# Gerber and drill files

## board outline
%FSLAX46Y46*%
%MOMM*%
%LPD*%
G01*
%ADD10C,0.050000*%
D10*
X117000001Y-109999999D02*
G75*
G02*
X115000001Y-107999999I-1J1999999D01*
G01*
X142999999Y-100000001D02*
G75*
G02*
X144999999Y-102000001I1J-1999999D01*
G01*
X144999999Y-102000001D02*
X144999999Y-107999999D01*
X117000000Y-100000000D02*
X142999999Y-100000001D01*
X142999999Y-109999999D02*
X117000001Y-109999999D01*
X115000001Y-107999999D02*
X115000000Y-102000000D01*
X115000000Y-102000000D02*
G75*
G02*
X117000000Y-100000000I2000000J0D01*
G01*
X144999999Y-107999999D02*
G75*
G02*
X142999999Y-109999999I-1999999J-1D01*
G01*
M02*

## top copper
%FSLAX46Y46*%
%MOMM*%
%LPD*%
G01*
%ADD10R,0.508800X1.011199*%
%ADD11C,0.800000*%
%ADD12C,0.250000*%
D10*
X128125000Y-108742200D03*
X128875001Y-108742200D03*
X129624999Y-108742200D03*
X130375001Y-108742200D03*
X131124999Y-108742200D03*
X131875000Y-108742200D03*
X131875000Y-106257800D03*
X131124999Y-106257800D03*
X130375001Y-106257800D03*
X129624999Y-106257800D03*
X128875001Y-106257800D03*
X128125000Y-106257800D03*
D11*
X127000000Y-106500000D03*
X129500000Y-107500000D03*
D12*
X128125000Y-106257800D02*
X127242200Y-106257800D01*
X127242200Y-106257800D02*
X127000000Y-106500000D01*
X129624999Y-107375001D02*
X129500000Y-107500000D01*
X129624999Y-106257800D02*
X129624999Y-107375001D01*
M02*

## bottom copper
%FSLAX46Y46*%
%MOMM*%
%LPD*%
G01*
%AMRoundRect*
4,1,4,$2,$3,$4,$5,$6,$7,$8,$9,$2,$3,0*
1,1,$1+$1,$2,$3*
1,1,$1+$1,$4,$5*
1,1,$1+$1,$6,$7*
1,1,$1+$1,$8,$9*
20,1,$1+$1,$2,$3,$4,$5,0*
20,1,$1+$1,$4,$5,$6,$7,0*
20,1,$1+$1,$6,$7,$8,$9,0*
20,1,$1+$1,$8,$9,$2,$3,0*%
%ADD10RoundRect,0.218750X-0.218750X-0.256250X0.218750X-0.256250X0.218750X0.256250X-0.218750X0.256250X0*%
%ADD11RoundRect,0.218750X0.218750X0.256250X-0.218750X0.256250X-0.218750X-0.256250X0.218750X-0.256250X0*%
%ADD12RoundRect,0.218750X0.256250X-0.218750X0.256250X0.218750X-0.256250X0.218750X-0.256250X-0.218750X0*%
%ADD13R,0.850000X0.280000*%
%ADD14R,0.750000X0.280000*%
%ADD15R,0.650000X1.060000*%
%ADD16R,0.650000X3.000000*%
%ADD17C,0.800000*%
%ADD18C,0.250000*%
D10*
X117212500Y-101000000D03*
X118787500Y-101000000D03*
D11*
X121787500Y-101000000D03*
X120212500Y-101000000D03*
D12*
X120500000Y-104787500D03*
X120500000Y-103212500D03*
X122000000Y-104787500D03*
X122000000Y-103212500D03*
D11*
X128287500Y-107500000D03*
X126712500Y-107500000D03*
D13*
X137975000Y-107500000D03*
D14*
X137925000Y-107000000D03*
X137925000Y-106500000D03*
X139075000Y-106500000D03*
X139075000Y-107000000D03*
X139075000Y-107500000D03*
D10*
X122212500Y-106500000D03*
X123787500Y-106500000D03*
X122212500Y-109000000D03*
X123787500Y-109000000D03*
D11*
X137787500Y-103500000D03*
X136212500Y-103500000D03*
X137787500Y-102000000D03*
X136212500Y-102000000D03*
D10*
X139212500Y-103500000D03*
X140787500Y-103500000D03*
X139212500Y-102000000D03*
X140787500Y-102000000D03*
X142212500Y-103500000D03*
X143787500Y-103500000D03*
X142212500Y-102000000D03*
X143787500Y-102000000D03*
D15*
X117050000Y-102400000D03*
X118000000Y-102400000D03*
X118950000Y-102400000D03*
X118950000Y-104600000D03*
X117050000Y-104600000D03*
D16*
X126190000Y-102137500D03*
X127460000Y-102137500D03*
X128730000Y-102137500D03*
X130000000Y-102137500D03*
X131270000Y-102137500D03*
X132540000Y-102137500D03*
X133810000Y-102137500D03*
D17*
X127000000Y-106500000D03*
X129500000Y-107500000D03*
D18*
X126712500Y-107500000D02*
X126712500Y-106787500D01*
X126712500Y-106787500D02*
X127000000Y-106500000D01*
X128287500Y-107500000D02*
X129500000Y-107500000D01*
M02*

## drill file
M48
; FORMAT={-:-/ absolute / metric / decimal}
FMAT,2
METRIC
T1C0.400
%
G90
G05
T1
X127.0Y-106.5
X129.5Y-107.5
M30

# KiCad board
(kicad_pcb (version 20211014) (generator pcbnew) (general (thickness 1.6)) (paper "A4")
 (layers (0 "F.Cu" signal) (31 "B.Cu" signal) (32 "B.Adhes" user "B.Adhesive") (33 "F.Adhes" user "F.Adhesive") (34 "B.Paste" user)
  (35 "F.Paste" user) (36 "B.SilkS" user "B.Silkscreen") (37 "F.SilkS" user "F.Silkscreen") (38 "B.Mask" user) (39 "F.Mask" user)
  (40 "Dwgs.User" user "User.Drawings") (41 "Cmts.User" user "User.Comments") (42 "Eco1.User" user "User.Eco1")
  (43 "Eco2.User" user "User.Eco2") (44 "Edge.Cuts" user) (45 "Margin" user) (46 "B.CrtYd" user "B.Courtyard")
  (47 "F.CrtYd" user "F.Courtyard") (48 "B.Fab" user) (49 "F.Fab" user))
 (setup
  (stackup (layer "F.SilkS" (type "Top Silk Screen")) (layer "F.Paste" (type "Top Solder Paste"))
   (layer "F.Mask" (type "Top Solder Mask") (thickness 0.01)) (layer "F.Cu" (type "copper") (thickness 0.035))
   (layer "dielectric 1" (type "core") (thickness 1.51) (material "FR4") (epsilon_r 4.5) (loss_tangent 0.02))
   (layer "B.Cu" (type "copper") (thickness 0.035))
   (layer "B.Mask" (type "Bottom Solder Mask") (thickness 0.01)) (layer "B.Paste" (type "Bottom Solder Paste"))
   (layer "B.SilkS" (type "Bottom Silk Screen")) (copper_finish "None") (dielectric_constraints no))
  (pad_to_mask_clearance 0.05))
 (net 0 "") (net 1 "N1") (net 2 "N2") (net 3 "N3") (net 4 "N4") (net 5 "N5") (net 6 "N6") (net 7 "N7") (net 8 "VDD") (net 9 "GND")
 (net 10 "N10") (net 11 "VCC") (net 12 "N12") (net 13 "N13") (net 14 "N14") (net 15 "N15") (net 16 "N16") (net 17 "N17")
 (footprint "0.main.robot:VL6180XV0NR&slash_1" (layer "F.Cu") (at 130 107.5 90)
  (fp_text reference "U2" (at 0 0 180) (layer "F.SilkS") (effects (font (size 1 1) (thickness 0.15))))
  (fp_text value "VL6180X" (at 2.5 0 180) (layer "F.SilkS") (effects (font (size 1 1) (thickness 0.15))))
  (pad "1" smd rect locked (at -1.2422 -1.875 90) (size 1.011199 0.5088) (layers "F.Cu" "F.Paste" "F.Mask") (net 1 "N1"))
  (pad "2" smd rect locked (at -1.2422 -1.124999 90) (size 1.011199 0.5088) (layers "F.Cu" "F.Paste" "F.Mask") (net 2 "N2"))
  (pad "3" smd rect locked (at -1.2422 -0.375001 90) (size 1.011199 0.5088) (layers "F.Cu" "F.Paste" "F.Mask") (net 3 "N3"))
  (pad "4" smd rect locked (at -1.2422 0.375001 90) (size 1.011199 0.5088) (layers "F.Cu" "F.Paste" "F.Mask") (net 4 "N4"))
  (pad "5" smd rect locked (at -1.2422 1.124999 90) (size 1.011199 0.5088) (layers "F.Cu" "F.Paste" "F.Mask") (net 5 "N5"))
  (pad "6" smd rect locked (at -1.2422 1.875 90) (size 1.011199 0.5088) (layers "F.Cu" "F.Paste" "F.Mask") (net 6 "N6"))
  (pad "7" smd rect locked (at 1.2422 1.875 90) (size 1.011199 0.5088) (layers "F.Cu" "F.Paste" "F.Mask") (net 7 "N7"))
  (pad "8" smd rect locked (at 1.2422 1.124999 90) (size 1.011199 0.5088) (layers "F.Cu" "F.Paste" "F.Mask") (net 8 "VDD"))
  (pad "9" smd rect locked (at 1.2422 0.375001 90) (size 1.011199 0.5088) (layers "F.Cu" "F.Paste" "F.Mask") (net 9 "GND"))
  (pad "10" smd rect locked (at 1.2422 -0.375001 90) (size 1.011199 0.5088) (layers "F.Cu" "F.Paste" "F.Mask") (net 8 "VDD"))
  (pad "11" smd rect locked (at 1.2422 -1.124999 90) (size 1.011199 0.5088) (layers "F.Cu" "F.Paste" "F.Mask") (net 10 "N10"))
  (pad "12" smd rect locked (at 1.2422 -1.875 90) (size 1.011199 0.5088) (layers "F.Cu" "F.Paste" "F.Mask") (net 9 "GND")))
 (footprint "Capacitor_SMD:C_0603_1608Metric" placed (layer "B.Cu") (at 118 101)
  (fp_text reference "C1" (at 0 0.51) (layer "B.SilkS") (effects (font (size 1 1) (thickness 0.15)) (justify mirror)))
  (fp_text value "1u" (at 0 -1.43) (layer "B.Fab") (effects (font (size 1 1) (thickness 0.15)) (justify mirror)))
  (pad "1" smd roundrect locked (at -0.7875 0) (size 0.875 0.95) (layers "B.Cu" "B.Paste" "B.Mask") (roundrect_rratio 0.25) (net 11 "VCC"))
  (pad "2" smd roundrect locked (at 0.7875 0) (size 0.875 0.95) (layers "B.Cu" "B.Paste" "B.Mask") (roundrect_rratio 0.25) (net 9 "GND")))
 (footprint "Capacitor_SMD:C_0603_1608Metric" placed (layer "B.Cu") (at 121 101 180)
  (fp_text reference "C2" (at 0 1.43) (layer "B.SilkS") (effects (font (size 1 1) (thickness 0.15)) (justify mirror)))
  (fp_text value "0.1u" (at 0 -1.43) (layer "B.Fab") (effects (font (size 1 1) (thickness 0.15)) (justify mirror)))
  (pad "1" smd roundrect locked (at -0.7875 0 180) (size 0.875 0.95) (layers "B.Cu" "B.Paste" "B.Mask") (roundrect_rratio 0.25)
   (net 11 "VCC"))
  (pad "2" smd roundrect locked (at 0.7875 0 180) (size 0.875 0.95) (layers "B.Cu" "B.Paste" "B.Mask") (roundrect_rratio 0.25) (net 9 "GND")))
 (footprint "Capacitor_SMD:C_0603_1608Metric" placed (layer "B.Cu") (at 120.5 104 90)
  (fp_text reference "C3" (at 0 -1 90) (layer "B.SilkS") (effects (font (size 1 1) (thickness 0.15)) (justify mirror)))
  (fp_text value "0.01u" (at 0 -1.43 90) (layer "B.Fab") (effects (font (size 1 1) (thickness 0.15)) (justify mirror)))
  (pad "1" smd roundrect locked (at -0.7875 0 90) (size 0.875 0.95) (layers "B.Cu" "B.Paste" "B.Mask") (roundrect_rratio 0.25)
   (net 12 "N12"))
  (pad "2" smd roundrect locked (at 0.7875 0 90) (size 0.875 0.95) (layers "B.Cu" "B.Paste" "B.Mask") (roundrect_rratio 0.25) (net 9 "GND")))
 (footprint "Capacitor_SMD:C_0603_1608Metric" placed (layer "B.Cu") (at 122 104 90)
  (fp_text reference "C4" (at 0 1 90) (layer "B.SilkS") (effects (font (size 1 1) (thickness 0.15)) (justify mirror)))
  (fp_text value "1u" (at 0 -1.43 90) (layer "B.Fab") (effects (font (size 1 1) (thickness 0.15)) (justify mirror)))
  (pad "1" smd roundrect locked (at -0.7875 0 90) (size 0.875 0.95) (layers "B.Cu" "B.Paste" "B.Mask") (roundrect_rratio 0.25) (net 8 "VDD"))
  (pad "2" smd roundrect locked (at 0.7875 0 90) (size 0.875 0.95) (layers "B.Cu" "B.Paste" "B.Mask") (roundrect_rratio 0.25) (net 9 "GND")))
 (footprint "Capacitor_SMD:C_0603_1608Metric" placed (layer "B.Cu") (at 127.5 107.5 180)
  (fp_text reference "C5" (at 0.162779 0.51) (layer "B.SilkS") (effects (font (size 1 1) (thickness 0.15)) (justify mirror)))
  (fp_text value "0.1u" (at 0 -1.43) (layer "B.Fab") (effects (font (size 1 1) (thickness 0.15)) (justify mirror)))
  (pad "1" smd roundrect locked (at -0.7875 0 180) (size 0.875 0.95) (layers "B.Cu" "B.Paste" "B.Mask") (roundrect_rratio 0.25)
   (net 8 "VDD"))
  (pad "2" smd roundrect locked (at 0.7875 0 180) (size 0.875 0.95) (layers "B.Cu" "B.Paste" "B.Mask") (roundrect_rratio 0.25) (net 9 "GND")))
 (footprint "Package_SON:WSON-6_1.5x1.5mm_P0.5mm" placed (layer "B.Cu") (at 138.5 107)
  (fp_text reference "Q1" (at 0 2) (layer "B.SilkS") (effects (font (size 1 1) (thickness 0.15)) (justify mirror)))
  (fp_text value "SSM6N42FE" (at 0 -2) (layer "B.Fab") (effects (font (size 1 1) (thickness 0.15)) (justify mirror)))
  (pad "1" smd rect locked (at -0.525 0.5 90) (size 0.28 0.85) (layers "B.Cu" "B.Paste" "B.Mask") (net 5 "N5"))
  (pad "2" smd rect locked (at -0.575 0 90) (size 0.28 0.75) (layers "B.Cu" "B.Paste" "B.Mask") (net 8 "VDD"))
  (pad "3" smd rect locked (at -0.575 -0.5 90) (size 0.28 0.75) (layers "B.Cu" "B.Paste" "B.Mask") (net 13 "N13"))
  (pad "4" smd rect locked (at 0.575 -0.5 90) (size 0.28 0.75) (layers "B.Cu" "B.Paste" "B.Mask") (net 6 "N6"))
  (pad "5" smd rect locked (at 0.575 0 90) (size 0.28 0.75) (layers "B.Cu" "B.Paste" "B.Mask") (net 8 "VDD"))
  (pad "6" smd rect locked (at 0.575 0.5 90) (size 0.28 0.75) (layers "B.Cu" "B.Paste" "B.Mask") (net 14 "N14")))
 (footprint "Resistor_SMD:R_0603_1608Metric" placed (layer "B.Cu") (at 123 106.5)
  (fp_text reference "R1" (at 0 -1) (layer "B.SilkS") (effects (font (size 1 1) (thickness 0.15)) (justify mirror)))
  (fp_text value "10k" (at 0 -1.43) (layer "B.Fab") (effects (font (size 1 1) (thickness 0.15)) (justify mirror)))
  (pad "1" smd roundrect locked (at -0.7875 0) (size 0.875 0.95) (layers "B.Cu" "B.Paste" "B.Mask") (roundrect_rratio 0.25) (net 11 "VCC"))
  (pad "2" smd roundrect locked (at 0.7875 0) (size 0.875 0.95) (layers "B.Cu" "B.Paste" "B.Mask") (roundrect_rratio 0.25) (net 14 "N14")))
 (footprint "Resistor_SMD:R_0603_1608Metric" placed (layer "B.Cu") (at 123 109)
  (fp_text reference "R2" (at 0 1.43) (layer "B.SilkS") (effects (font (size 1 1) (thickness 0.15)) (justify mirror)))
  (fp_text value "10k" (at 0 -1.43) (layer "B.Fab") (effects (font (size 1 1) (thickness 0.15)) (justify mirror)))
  (pad "1" smd roundrect locked (at -0.7875 0) (size 0.875 0.95) (layers "B.Cu" "B.Paste" "B.Mask") (roundrect_rratio 0.25) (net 11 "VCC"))
  (pad "2" smd roundrect locked (at 0.7875 0) (size 0.875 0.95) (layers "B.Cu" "B.Paste" "B.Mask") (roundrect_rratio 0.25) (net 13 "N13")))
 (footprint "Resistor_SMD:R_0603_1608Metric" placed (layer "B.Cu") (at 137 103.5 180)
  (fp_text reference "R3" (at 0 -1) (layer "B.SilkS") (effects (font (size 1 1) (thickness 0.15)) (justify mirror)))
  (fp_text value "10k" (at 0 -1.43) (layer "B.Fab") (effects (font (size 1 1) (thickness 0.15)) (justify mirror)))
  (pad "1" smd roundrect locked (at -0.7875 0 180) (size 0.875 0.95) (layers "B.Cu" "B.Paste" "B.Mask") (roundrect_rratio 0.25)
   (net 8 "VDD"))
  (pad "2" smd roundrect locked (at 0.7875 0 180) (size 0.875 0.95) (layers "B.Cu" "B.Paste" "B.Mask") (roundrect_rratio 0.25) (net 5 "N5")))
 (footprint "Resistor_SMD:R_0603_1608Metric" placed (layer "B.Cu") (at 137 102 180)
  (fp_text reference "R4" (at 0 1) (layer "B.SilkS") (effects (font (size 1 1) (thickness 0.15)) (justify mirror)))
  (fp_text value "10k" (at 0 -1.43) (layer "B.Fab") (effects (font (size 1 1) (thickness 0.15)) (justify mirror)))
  (pad "1" smd roundrect locked (at -0.7875 0 180) (size 0.875 0.95) (layers "B.Cu" "B.Paste" "B.Mask") (roundrect_rratio 0.25)
   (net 8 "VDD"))
  (pad "2" smd roundrect locked (at 0.7875 0 180) (size 0.875 0.95) (layers "B.Cu" "B.Paste" "B.Mask") (roundrect_rratio 0.25) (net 6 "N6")))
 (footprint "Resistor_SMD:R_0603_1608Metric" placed (layer "B.Cu") (at 140 103.5)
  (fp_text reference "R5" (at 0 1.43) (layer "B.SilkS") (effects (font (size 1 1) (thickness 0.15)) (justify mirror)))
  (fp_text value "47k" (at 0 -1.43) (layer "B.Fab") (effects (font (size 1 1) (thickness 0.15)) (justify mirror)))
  (pad "1" smd roundrect locked (at -0.7875 0) (size 0.875 0.95) (layers "B.Cu" "B.Paste" "B.Mask") (roundrect_rratio 0.25) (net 8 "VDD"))
  (pad "2" smd roundrect locked (at 0.7875 0) (size 0.875 0.95) (layers "B.Cu" "B.Paste" "B.Mask") (roundrect_rratio 0.25) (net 4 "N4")))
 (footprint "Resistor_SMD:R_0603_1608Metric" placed (layer "B.Cu") (at 140 102)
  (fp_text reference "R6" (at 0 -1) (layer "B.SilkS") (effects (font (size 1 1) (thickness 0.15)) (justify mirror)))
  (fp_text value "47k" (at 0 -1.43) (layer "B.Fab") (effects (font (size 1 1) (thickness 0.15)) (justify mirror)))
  (pad "1" smd roundrect locked (at -0.7875 0) (size 0.875 0.95) (layers "B.Cu" "B.Paste" "B.Mask") (roundrect_rratio 0.25) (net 8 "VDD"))
  (pad "2" smd roundrect locked (at 0.7875 0) (size 0.875 0.95) (layers "B.Cu" "B.Paste" "B.Mask") (roundrect_rratio 0.25) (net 1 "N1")))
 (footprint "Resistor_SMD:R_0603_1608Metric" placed (layer "B.Cu") (at 143 103.5)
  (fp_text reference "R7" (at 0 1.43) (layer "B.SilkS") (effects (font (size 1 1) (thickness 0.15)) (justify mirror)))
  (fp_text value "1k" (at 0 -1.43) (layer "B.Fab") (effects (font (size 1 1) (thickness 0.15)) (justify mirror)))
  (pad "1" smd roundrect locked (at -0.7875 0) (size 0.875 0.95) (layers "B.Cu" "B.Paste" "B.Mask") (roundrect_rratio 0.25) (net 4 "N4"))
  (pad "2" smd roundrect locked (at 0.7875 0) (size 0.875 0.95) (layers "B.Cu" "B.Paste" "B.Mask") (roundrect_rratio 0.25) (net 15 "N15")))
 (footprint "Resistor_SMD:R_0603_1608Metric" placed (layer "B.Cu") (at 143 102)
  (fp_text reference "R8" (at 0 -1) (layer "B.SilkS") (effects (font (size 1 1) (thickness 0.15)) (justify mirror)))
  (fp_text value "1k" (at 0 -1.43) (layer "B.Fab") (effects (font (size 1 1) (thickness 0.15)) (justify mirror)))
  (pad "1" smd roundrect locked (at -0.7875 0) (size 0.875 0.95) (layers "B.Cu" "B.Paste" "B.Mask") (roundrect_rratio 0.25) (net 1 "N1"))
  (pad "2" smd roundrect locked (at 0.7875 0) (size 0.875 0.95) (layers "B.Cu" "B.Paste" "B.Mask") (roundrect_rratio 0.25) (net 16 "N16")))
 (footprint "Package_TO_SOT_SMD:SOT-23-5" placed (layer "B.Cu") (at 118 103.5 -90)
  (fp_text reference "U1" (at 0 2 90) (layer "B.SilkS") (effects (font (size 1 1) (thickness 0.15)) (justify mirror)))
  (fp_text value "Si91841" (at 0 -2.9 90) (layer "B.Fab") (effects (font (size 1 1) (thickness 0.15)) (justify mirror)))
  (pad "1" smd rect locked (at -1.1 0.95 270) (size 1.06 0.65) (layers "B.Cu" "B.Paste" "B.Mask") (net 11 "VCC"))
  (pad "2" smd rect locked (at -1.1 0 270) (size 1.06 0.65) (layers "B.Cu" "B.Paste" "B.Mask") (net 9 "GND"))
  (pad "3" smd rect locked (at -1.1 -0.95 270) (size 1.06 0.65) (layers "B.Cu" "B.Paste" "B.Mask") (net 11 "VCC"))
  (pad "4" smd rect locked (at 1.1 -0.95 270) (size 1.06 0.65) (layers "B.Cu" "B.Paste" "B.Mask") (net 12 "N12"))
  (pad "5" smd rect locked (at 1.1 0.95 270) (size 1.06 0.65) (layers "B.Cu" "B.Paste" "B.Mask") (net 8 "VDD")))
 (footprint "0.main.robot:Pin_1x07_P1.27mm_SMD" (layer "B.Cu") (at 130 103.6375 -90)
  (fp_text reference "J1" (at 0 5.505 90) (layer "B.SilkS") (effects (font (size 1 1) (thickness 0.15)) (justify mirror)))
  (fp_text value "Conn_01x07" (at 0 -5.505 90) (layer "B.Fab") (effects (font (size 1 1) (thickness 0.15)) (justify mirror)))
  (pad "1" smd rect locked (at -1.5 3.81 270) (size 3 0.65) (layers "B.Cu" "B.Paste" "B.Mask") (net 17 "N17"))
  (pad "2" smd rect locked (at -1.5 2.54 270) (size 3 0.65) (layers "B.Cu" "B.Paste" "B.Mask") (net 11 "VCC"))
  (pad "3" smd rect locked (at -1.5 1.27 270) (size 3 0.65) (layers "B.Cu" "B.Paste" "B.Mask") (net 9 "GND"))
  (pad "4" smd rect locked (at -1.5 0 270) (size 3 0.65) (layers "B.Cu" "B.Paste" "B.Mask") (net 13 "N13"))
  (pad "5" smd rect locked (at -1.5 -1.27 270) (size 3 0.65) (layers "B.Cu" "B.Paste" "B.Mask") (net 14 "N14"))
  (pad "6" smd rect locked (at -1.5 -2.54 270) (size 3 0.65) (layers "B.Cu" "B.Paste" "B.Mask") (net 15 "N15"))
  (pad "7" smd rect locked (at -1.5 -3.81 270) (size 3 0.65) (layers "B.Cu" "B.Paste" "B.Mask") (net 16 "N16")))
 (gr_arc (start 117.000001 109.999999) (mid 115.585787 109.414213) (end 115.000001 107.999999) (layer "Edge.Cuts") (width 0.05))
 (gr_arc (start 142.999999 100.000001) (mid 144.414213 100.585787) (end 144.999999 102.000001) (layer "Edge.Cuts") (width 0.05))
 (gr_line (start 144.999999 102.000001) (end 144.999999 107.999999) (layer "Edge.Cuts") (width 0.05))
 (gr_line (start 117 100) (end 142.999999 100.000001) (layer "Edge.Cuts") (width 0.05))
 (gr_line (start 142.999999 109.999999) (end 117.000001 109.999999) (layer "Edge.Cuts") (width 0.05))
 (gr_line (start 115.000001 107.999999) (end 115 102) (layer "Edge.Cuts") (width 0.05))
 (gr_arc (start 115 102) (mid 115.585786 100.585786) (end 117 100) (layer "Edge.Cuts") (width 0.05))
 (gr_arc (start 144.999999 107.999999) (mid 144.414213 109.414213) (end 142.999999 109.999999) (layer "Edge.Cuts") (width 0.05))
 (segment (start 128.125 106.2578) (end 127.2422 106.2578) (width 0.25) (layer "F.Cu") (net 9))
 (segment (start 127.2422 106.2578) (end 127 106.5) (width 0.25) (layer "F.Cu") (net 9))
 (via (at 127 106.5) (size 0.8) (drill 0.4) (layers "F.Cu" "B.Cu") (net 9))
 (segment (start 126.7125 107.5) (end 126.7125 106.7875) (width 0.25) (layer "B.Cu") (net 9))
 (segment (start 126.7125 106.7875) (end 127 106.5) (width 0.25) (layer "B.Cu") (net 9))
 (segment (start 129.624999 107.375001) (end 129.5 107.5) (width 0.25) (layer "F.Cu") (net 8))
 (segment (start 129.624999 106.2578) (end 129.624999 107.375001) (width 0.25) (layer "F.Cu") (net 8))
 (via (at 129.5 107.5) (size 0.8) (drill 0.4) (layers "F.Cu" "B.Cu") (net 8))
 (segment (start 128.2875 107.5) (end 129.5 107.5) (width 0.25) (layer "B.Cu") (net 8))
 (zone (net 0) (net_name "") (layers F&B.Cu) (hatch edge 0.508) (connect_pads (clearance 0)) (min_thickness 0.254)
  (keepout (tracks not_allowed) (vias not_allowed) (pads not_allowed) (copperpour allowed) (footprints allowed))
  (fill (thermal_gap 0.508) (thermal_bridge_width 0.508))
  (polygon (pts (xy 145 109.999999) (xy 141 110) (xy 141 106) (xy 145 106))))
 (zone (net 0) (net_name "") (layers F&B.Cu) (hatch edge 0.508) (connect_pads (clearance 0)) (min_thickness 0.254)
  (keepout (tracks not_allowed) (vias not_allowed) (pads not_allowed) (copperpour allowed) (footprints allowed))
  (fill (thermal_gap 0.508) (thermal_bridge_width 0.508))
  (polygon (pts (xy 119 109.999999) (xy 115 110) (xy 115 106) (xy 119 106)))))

